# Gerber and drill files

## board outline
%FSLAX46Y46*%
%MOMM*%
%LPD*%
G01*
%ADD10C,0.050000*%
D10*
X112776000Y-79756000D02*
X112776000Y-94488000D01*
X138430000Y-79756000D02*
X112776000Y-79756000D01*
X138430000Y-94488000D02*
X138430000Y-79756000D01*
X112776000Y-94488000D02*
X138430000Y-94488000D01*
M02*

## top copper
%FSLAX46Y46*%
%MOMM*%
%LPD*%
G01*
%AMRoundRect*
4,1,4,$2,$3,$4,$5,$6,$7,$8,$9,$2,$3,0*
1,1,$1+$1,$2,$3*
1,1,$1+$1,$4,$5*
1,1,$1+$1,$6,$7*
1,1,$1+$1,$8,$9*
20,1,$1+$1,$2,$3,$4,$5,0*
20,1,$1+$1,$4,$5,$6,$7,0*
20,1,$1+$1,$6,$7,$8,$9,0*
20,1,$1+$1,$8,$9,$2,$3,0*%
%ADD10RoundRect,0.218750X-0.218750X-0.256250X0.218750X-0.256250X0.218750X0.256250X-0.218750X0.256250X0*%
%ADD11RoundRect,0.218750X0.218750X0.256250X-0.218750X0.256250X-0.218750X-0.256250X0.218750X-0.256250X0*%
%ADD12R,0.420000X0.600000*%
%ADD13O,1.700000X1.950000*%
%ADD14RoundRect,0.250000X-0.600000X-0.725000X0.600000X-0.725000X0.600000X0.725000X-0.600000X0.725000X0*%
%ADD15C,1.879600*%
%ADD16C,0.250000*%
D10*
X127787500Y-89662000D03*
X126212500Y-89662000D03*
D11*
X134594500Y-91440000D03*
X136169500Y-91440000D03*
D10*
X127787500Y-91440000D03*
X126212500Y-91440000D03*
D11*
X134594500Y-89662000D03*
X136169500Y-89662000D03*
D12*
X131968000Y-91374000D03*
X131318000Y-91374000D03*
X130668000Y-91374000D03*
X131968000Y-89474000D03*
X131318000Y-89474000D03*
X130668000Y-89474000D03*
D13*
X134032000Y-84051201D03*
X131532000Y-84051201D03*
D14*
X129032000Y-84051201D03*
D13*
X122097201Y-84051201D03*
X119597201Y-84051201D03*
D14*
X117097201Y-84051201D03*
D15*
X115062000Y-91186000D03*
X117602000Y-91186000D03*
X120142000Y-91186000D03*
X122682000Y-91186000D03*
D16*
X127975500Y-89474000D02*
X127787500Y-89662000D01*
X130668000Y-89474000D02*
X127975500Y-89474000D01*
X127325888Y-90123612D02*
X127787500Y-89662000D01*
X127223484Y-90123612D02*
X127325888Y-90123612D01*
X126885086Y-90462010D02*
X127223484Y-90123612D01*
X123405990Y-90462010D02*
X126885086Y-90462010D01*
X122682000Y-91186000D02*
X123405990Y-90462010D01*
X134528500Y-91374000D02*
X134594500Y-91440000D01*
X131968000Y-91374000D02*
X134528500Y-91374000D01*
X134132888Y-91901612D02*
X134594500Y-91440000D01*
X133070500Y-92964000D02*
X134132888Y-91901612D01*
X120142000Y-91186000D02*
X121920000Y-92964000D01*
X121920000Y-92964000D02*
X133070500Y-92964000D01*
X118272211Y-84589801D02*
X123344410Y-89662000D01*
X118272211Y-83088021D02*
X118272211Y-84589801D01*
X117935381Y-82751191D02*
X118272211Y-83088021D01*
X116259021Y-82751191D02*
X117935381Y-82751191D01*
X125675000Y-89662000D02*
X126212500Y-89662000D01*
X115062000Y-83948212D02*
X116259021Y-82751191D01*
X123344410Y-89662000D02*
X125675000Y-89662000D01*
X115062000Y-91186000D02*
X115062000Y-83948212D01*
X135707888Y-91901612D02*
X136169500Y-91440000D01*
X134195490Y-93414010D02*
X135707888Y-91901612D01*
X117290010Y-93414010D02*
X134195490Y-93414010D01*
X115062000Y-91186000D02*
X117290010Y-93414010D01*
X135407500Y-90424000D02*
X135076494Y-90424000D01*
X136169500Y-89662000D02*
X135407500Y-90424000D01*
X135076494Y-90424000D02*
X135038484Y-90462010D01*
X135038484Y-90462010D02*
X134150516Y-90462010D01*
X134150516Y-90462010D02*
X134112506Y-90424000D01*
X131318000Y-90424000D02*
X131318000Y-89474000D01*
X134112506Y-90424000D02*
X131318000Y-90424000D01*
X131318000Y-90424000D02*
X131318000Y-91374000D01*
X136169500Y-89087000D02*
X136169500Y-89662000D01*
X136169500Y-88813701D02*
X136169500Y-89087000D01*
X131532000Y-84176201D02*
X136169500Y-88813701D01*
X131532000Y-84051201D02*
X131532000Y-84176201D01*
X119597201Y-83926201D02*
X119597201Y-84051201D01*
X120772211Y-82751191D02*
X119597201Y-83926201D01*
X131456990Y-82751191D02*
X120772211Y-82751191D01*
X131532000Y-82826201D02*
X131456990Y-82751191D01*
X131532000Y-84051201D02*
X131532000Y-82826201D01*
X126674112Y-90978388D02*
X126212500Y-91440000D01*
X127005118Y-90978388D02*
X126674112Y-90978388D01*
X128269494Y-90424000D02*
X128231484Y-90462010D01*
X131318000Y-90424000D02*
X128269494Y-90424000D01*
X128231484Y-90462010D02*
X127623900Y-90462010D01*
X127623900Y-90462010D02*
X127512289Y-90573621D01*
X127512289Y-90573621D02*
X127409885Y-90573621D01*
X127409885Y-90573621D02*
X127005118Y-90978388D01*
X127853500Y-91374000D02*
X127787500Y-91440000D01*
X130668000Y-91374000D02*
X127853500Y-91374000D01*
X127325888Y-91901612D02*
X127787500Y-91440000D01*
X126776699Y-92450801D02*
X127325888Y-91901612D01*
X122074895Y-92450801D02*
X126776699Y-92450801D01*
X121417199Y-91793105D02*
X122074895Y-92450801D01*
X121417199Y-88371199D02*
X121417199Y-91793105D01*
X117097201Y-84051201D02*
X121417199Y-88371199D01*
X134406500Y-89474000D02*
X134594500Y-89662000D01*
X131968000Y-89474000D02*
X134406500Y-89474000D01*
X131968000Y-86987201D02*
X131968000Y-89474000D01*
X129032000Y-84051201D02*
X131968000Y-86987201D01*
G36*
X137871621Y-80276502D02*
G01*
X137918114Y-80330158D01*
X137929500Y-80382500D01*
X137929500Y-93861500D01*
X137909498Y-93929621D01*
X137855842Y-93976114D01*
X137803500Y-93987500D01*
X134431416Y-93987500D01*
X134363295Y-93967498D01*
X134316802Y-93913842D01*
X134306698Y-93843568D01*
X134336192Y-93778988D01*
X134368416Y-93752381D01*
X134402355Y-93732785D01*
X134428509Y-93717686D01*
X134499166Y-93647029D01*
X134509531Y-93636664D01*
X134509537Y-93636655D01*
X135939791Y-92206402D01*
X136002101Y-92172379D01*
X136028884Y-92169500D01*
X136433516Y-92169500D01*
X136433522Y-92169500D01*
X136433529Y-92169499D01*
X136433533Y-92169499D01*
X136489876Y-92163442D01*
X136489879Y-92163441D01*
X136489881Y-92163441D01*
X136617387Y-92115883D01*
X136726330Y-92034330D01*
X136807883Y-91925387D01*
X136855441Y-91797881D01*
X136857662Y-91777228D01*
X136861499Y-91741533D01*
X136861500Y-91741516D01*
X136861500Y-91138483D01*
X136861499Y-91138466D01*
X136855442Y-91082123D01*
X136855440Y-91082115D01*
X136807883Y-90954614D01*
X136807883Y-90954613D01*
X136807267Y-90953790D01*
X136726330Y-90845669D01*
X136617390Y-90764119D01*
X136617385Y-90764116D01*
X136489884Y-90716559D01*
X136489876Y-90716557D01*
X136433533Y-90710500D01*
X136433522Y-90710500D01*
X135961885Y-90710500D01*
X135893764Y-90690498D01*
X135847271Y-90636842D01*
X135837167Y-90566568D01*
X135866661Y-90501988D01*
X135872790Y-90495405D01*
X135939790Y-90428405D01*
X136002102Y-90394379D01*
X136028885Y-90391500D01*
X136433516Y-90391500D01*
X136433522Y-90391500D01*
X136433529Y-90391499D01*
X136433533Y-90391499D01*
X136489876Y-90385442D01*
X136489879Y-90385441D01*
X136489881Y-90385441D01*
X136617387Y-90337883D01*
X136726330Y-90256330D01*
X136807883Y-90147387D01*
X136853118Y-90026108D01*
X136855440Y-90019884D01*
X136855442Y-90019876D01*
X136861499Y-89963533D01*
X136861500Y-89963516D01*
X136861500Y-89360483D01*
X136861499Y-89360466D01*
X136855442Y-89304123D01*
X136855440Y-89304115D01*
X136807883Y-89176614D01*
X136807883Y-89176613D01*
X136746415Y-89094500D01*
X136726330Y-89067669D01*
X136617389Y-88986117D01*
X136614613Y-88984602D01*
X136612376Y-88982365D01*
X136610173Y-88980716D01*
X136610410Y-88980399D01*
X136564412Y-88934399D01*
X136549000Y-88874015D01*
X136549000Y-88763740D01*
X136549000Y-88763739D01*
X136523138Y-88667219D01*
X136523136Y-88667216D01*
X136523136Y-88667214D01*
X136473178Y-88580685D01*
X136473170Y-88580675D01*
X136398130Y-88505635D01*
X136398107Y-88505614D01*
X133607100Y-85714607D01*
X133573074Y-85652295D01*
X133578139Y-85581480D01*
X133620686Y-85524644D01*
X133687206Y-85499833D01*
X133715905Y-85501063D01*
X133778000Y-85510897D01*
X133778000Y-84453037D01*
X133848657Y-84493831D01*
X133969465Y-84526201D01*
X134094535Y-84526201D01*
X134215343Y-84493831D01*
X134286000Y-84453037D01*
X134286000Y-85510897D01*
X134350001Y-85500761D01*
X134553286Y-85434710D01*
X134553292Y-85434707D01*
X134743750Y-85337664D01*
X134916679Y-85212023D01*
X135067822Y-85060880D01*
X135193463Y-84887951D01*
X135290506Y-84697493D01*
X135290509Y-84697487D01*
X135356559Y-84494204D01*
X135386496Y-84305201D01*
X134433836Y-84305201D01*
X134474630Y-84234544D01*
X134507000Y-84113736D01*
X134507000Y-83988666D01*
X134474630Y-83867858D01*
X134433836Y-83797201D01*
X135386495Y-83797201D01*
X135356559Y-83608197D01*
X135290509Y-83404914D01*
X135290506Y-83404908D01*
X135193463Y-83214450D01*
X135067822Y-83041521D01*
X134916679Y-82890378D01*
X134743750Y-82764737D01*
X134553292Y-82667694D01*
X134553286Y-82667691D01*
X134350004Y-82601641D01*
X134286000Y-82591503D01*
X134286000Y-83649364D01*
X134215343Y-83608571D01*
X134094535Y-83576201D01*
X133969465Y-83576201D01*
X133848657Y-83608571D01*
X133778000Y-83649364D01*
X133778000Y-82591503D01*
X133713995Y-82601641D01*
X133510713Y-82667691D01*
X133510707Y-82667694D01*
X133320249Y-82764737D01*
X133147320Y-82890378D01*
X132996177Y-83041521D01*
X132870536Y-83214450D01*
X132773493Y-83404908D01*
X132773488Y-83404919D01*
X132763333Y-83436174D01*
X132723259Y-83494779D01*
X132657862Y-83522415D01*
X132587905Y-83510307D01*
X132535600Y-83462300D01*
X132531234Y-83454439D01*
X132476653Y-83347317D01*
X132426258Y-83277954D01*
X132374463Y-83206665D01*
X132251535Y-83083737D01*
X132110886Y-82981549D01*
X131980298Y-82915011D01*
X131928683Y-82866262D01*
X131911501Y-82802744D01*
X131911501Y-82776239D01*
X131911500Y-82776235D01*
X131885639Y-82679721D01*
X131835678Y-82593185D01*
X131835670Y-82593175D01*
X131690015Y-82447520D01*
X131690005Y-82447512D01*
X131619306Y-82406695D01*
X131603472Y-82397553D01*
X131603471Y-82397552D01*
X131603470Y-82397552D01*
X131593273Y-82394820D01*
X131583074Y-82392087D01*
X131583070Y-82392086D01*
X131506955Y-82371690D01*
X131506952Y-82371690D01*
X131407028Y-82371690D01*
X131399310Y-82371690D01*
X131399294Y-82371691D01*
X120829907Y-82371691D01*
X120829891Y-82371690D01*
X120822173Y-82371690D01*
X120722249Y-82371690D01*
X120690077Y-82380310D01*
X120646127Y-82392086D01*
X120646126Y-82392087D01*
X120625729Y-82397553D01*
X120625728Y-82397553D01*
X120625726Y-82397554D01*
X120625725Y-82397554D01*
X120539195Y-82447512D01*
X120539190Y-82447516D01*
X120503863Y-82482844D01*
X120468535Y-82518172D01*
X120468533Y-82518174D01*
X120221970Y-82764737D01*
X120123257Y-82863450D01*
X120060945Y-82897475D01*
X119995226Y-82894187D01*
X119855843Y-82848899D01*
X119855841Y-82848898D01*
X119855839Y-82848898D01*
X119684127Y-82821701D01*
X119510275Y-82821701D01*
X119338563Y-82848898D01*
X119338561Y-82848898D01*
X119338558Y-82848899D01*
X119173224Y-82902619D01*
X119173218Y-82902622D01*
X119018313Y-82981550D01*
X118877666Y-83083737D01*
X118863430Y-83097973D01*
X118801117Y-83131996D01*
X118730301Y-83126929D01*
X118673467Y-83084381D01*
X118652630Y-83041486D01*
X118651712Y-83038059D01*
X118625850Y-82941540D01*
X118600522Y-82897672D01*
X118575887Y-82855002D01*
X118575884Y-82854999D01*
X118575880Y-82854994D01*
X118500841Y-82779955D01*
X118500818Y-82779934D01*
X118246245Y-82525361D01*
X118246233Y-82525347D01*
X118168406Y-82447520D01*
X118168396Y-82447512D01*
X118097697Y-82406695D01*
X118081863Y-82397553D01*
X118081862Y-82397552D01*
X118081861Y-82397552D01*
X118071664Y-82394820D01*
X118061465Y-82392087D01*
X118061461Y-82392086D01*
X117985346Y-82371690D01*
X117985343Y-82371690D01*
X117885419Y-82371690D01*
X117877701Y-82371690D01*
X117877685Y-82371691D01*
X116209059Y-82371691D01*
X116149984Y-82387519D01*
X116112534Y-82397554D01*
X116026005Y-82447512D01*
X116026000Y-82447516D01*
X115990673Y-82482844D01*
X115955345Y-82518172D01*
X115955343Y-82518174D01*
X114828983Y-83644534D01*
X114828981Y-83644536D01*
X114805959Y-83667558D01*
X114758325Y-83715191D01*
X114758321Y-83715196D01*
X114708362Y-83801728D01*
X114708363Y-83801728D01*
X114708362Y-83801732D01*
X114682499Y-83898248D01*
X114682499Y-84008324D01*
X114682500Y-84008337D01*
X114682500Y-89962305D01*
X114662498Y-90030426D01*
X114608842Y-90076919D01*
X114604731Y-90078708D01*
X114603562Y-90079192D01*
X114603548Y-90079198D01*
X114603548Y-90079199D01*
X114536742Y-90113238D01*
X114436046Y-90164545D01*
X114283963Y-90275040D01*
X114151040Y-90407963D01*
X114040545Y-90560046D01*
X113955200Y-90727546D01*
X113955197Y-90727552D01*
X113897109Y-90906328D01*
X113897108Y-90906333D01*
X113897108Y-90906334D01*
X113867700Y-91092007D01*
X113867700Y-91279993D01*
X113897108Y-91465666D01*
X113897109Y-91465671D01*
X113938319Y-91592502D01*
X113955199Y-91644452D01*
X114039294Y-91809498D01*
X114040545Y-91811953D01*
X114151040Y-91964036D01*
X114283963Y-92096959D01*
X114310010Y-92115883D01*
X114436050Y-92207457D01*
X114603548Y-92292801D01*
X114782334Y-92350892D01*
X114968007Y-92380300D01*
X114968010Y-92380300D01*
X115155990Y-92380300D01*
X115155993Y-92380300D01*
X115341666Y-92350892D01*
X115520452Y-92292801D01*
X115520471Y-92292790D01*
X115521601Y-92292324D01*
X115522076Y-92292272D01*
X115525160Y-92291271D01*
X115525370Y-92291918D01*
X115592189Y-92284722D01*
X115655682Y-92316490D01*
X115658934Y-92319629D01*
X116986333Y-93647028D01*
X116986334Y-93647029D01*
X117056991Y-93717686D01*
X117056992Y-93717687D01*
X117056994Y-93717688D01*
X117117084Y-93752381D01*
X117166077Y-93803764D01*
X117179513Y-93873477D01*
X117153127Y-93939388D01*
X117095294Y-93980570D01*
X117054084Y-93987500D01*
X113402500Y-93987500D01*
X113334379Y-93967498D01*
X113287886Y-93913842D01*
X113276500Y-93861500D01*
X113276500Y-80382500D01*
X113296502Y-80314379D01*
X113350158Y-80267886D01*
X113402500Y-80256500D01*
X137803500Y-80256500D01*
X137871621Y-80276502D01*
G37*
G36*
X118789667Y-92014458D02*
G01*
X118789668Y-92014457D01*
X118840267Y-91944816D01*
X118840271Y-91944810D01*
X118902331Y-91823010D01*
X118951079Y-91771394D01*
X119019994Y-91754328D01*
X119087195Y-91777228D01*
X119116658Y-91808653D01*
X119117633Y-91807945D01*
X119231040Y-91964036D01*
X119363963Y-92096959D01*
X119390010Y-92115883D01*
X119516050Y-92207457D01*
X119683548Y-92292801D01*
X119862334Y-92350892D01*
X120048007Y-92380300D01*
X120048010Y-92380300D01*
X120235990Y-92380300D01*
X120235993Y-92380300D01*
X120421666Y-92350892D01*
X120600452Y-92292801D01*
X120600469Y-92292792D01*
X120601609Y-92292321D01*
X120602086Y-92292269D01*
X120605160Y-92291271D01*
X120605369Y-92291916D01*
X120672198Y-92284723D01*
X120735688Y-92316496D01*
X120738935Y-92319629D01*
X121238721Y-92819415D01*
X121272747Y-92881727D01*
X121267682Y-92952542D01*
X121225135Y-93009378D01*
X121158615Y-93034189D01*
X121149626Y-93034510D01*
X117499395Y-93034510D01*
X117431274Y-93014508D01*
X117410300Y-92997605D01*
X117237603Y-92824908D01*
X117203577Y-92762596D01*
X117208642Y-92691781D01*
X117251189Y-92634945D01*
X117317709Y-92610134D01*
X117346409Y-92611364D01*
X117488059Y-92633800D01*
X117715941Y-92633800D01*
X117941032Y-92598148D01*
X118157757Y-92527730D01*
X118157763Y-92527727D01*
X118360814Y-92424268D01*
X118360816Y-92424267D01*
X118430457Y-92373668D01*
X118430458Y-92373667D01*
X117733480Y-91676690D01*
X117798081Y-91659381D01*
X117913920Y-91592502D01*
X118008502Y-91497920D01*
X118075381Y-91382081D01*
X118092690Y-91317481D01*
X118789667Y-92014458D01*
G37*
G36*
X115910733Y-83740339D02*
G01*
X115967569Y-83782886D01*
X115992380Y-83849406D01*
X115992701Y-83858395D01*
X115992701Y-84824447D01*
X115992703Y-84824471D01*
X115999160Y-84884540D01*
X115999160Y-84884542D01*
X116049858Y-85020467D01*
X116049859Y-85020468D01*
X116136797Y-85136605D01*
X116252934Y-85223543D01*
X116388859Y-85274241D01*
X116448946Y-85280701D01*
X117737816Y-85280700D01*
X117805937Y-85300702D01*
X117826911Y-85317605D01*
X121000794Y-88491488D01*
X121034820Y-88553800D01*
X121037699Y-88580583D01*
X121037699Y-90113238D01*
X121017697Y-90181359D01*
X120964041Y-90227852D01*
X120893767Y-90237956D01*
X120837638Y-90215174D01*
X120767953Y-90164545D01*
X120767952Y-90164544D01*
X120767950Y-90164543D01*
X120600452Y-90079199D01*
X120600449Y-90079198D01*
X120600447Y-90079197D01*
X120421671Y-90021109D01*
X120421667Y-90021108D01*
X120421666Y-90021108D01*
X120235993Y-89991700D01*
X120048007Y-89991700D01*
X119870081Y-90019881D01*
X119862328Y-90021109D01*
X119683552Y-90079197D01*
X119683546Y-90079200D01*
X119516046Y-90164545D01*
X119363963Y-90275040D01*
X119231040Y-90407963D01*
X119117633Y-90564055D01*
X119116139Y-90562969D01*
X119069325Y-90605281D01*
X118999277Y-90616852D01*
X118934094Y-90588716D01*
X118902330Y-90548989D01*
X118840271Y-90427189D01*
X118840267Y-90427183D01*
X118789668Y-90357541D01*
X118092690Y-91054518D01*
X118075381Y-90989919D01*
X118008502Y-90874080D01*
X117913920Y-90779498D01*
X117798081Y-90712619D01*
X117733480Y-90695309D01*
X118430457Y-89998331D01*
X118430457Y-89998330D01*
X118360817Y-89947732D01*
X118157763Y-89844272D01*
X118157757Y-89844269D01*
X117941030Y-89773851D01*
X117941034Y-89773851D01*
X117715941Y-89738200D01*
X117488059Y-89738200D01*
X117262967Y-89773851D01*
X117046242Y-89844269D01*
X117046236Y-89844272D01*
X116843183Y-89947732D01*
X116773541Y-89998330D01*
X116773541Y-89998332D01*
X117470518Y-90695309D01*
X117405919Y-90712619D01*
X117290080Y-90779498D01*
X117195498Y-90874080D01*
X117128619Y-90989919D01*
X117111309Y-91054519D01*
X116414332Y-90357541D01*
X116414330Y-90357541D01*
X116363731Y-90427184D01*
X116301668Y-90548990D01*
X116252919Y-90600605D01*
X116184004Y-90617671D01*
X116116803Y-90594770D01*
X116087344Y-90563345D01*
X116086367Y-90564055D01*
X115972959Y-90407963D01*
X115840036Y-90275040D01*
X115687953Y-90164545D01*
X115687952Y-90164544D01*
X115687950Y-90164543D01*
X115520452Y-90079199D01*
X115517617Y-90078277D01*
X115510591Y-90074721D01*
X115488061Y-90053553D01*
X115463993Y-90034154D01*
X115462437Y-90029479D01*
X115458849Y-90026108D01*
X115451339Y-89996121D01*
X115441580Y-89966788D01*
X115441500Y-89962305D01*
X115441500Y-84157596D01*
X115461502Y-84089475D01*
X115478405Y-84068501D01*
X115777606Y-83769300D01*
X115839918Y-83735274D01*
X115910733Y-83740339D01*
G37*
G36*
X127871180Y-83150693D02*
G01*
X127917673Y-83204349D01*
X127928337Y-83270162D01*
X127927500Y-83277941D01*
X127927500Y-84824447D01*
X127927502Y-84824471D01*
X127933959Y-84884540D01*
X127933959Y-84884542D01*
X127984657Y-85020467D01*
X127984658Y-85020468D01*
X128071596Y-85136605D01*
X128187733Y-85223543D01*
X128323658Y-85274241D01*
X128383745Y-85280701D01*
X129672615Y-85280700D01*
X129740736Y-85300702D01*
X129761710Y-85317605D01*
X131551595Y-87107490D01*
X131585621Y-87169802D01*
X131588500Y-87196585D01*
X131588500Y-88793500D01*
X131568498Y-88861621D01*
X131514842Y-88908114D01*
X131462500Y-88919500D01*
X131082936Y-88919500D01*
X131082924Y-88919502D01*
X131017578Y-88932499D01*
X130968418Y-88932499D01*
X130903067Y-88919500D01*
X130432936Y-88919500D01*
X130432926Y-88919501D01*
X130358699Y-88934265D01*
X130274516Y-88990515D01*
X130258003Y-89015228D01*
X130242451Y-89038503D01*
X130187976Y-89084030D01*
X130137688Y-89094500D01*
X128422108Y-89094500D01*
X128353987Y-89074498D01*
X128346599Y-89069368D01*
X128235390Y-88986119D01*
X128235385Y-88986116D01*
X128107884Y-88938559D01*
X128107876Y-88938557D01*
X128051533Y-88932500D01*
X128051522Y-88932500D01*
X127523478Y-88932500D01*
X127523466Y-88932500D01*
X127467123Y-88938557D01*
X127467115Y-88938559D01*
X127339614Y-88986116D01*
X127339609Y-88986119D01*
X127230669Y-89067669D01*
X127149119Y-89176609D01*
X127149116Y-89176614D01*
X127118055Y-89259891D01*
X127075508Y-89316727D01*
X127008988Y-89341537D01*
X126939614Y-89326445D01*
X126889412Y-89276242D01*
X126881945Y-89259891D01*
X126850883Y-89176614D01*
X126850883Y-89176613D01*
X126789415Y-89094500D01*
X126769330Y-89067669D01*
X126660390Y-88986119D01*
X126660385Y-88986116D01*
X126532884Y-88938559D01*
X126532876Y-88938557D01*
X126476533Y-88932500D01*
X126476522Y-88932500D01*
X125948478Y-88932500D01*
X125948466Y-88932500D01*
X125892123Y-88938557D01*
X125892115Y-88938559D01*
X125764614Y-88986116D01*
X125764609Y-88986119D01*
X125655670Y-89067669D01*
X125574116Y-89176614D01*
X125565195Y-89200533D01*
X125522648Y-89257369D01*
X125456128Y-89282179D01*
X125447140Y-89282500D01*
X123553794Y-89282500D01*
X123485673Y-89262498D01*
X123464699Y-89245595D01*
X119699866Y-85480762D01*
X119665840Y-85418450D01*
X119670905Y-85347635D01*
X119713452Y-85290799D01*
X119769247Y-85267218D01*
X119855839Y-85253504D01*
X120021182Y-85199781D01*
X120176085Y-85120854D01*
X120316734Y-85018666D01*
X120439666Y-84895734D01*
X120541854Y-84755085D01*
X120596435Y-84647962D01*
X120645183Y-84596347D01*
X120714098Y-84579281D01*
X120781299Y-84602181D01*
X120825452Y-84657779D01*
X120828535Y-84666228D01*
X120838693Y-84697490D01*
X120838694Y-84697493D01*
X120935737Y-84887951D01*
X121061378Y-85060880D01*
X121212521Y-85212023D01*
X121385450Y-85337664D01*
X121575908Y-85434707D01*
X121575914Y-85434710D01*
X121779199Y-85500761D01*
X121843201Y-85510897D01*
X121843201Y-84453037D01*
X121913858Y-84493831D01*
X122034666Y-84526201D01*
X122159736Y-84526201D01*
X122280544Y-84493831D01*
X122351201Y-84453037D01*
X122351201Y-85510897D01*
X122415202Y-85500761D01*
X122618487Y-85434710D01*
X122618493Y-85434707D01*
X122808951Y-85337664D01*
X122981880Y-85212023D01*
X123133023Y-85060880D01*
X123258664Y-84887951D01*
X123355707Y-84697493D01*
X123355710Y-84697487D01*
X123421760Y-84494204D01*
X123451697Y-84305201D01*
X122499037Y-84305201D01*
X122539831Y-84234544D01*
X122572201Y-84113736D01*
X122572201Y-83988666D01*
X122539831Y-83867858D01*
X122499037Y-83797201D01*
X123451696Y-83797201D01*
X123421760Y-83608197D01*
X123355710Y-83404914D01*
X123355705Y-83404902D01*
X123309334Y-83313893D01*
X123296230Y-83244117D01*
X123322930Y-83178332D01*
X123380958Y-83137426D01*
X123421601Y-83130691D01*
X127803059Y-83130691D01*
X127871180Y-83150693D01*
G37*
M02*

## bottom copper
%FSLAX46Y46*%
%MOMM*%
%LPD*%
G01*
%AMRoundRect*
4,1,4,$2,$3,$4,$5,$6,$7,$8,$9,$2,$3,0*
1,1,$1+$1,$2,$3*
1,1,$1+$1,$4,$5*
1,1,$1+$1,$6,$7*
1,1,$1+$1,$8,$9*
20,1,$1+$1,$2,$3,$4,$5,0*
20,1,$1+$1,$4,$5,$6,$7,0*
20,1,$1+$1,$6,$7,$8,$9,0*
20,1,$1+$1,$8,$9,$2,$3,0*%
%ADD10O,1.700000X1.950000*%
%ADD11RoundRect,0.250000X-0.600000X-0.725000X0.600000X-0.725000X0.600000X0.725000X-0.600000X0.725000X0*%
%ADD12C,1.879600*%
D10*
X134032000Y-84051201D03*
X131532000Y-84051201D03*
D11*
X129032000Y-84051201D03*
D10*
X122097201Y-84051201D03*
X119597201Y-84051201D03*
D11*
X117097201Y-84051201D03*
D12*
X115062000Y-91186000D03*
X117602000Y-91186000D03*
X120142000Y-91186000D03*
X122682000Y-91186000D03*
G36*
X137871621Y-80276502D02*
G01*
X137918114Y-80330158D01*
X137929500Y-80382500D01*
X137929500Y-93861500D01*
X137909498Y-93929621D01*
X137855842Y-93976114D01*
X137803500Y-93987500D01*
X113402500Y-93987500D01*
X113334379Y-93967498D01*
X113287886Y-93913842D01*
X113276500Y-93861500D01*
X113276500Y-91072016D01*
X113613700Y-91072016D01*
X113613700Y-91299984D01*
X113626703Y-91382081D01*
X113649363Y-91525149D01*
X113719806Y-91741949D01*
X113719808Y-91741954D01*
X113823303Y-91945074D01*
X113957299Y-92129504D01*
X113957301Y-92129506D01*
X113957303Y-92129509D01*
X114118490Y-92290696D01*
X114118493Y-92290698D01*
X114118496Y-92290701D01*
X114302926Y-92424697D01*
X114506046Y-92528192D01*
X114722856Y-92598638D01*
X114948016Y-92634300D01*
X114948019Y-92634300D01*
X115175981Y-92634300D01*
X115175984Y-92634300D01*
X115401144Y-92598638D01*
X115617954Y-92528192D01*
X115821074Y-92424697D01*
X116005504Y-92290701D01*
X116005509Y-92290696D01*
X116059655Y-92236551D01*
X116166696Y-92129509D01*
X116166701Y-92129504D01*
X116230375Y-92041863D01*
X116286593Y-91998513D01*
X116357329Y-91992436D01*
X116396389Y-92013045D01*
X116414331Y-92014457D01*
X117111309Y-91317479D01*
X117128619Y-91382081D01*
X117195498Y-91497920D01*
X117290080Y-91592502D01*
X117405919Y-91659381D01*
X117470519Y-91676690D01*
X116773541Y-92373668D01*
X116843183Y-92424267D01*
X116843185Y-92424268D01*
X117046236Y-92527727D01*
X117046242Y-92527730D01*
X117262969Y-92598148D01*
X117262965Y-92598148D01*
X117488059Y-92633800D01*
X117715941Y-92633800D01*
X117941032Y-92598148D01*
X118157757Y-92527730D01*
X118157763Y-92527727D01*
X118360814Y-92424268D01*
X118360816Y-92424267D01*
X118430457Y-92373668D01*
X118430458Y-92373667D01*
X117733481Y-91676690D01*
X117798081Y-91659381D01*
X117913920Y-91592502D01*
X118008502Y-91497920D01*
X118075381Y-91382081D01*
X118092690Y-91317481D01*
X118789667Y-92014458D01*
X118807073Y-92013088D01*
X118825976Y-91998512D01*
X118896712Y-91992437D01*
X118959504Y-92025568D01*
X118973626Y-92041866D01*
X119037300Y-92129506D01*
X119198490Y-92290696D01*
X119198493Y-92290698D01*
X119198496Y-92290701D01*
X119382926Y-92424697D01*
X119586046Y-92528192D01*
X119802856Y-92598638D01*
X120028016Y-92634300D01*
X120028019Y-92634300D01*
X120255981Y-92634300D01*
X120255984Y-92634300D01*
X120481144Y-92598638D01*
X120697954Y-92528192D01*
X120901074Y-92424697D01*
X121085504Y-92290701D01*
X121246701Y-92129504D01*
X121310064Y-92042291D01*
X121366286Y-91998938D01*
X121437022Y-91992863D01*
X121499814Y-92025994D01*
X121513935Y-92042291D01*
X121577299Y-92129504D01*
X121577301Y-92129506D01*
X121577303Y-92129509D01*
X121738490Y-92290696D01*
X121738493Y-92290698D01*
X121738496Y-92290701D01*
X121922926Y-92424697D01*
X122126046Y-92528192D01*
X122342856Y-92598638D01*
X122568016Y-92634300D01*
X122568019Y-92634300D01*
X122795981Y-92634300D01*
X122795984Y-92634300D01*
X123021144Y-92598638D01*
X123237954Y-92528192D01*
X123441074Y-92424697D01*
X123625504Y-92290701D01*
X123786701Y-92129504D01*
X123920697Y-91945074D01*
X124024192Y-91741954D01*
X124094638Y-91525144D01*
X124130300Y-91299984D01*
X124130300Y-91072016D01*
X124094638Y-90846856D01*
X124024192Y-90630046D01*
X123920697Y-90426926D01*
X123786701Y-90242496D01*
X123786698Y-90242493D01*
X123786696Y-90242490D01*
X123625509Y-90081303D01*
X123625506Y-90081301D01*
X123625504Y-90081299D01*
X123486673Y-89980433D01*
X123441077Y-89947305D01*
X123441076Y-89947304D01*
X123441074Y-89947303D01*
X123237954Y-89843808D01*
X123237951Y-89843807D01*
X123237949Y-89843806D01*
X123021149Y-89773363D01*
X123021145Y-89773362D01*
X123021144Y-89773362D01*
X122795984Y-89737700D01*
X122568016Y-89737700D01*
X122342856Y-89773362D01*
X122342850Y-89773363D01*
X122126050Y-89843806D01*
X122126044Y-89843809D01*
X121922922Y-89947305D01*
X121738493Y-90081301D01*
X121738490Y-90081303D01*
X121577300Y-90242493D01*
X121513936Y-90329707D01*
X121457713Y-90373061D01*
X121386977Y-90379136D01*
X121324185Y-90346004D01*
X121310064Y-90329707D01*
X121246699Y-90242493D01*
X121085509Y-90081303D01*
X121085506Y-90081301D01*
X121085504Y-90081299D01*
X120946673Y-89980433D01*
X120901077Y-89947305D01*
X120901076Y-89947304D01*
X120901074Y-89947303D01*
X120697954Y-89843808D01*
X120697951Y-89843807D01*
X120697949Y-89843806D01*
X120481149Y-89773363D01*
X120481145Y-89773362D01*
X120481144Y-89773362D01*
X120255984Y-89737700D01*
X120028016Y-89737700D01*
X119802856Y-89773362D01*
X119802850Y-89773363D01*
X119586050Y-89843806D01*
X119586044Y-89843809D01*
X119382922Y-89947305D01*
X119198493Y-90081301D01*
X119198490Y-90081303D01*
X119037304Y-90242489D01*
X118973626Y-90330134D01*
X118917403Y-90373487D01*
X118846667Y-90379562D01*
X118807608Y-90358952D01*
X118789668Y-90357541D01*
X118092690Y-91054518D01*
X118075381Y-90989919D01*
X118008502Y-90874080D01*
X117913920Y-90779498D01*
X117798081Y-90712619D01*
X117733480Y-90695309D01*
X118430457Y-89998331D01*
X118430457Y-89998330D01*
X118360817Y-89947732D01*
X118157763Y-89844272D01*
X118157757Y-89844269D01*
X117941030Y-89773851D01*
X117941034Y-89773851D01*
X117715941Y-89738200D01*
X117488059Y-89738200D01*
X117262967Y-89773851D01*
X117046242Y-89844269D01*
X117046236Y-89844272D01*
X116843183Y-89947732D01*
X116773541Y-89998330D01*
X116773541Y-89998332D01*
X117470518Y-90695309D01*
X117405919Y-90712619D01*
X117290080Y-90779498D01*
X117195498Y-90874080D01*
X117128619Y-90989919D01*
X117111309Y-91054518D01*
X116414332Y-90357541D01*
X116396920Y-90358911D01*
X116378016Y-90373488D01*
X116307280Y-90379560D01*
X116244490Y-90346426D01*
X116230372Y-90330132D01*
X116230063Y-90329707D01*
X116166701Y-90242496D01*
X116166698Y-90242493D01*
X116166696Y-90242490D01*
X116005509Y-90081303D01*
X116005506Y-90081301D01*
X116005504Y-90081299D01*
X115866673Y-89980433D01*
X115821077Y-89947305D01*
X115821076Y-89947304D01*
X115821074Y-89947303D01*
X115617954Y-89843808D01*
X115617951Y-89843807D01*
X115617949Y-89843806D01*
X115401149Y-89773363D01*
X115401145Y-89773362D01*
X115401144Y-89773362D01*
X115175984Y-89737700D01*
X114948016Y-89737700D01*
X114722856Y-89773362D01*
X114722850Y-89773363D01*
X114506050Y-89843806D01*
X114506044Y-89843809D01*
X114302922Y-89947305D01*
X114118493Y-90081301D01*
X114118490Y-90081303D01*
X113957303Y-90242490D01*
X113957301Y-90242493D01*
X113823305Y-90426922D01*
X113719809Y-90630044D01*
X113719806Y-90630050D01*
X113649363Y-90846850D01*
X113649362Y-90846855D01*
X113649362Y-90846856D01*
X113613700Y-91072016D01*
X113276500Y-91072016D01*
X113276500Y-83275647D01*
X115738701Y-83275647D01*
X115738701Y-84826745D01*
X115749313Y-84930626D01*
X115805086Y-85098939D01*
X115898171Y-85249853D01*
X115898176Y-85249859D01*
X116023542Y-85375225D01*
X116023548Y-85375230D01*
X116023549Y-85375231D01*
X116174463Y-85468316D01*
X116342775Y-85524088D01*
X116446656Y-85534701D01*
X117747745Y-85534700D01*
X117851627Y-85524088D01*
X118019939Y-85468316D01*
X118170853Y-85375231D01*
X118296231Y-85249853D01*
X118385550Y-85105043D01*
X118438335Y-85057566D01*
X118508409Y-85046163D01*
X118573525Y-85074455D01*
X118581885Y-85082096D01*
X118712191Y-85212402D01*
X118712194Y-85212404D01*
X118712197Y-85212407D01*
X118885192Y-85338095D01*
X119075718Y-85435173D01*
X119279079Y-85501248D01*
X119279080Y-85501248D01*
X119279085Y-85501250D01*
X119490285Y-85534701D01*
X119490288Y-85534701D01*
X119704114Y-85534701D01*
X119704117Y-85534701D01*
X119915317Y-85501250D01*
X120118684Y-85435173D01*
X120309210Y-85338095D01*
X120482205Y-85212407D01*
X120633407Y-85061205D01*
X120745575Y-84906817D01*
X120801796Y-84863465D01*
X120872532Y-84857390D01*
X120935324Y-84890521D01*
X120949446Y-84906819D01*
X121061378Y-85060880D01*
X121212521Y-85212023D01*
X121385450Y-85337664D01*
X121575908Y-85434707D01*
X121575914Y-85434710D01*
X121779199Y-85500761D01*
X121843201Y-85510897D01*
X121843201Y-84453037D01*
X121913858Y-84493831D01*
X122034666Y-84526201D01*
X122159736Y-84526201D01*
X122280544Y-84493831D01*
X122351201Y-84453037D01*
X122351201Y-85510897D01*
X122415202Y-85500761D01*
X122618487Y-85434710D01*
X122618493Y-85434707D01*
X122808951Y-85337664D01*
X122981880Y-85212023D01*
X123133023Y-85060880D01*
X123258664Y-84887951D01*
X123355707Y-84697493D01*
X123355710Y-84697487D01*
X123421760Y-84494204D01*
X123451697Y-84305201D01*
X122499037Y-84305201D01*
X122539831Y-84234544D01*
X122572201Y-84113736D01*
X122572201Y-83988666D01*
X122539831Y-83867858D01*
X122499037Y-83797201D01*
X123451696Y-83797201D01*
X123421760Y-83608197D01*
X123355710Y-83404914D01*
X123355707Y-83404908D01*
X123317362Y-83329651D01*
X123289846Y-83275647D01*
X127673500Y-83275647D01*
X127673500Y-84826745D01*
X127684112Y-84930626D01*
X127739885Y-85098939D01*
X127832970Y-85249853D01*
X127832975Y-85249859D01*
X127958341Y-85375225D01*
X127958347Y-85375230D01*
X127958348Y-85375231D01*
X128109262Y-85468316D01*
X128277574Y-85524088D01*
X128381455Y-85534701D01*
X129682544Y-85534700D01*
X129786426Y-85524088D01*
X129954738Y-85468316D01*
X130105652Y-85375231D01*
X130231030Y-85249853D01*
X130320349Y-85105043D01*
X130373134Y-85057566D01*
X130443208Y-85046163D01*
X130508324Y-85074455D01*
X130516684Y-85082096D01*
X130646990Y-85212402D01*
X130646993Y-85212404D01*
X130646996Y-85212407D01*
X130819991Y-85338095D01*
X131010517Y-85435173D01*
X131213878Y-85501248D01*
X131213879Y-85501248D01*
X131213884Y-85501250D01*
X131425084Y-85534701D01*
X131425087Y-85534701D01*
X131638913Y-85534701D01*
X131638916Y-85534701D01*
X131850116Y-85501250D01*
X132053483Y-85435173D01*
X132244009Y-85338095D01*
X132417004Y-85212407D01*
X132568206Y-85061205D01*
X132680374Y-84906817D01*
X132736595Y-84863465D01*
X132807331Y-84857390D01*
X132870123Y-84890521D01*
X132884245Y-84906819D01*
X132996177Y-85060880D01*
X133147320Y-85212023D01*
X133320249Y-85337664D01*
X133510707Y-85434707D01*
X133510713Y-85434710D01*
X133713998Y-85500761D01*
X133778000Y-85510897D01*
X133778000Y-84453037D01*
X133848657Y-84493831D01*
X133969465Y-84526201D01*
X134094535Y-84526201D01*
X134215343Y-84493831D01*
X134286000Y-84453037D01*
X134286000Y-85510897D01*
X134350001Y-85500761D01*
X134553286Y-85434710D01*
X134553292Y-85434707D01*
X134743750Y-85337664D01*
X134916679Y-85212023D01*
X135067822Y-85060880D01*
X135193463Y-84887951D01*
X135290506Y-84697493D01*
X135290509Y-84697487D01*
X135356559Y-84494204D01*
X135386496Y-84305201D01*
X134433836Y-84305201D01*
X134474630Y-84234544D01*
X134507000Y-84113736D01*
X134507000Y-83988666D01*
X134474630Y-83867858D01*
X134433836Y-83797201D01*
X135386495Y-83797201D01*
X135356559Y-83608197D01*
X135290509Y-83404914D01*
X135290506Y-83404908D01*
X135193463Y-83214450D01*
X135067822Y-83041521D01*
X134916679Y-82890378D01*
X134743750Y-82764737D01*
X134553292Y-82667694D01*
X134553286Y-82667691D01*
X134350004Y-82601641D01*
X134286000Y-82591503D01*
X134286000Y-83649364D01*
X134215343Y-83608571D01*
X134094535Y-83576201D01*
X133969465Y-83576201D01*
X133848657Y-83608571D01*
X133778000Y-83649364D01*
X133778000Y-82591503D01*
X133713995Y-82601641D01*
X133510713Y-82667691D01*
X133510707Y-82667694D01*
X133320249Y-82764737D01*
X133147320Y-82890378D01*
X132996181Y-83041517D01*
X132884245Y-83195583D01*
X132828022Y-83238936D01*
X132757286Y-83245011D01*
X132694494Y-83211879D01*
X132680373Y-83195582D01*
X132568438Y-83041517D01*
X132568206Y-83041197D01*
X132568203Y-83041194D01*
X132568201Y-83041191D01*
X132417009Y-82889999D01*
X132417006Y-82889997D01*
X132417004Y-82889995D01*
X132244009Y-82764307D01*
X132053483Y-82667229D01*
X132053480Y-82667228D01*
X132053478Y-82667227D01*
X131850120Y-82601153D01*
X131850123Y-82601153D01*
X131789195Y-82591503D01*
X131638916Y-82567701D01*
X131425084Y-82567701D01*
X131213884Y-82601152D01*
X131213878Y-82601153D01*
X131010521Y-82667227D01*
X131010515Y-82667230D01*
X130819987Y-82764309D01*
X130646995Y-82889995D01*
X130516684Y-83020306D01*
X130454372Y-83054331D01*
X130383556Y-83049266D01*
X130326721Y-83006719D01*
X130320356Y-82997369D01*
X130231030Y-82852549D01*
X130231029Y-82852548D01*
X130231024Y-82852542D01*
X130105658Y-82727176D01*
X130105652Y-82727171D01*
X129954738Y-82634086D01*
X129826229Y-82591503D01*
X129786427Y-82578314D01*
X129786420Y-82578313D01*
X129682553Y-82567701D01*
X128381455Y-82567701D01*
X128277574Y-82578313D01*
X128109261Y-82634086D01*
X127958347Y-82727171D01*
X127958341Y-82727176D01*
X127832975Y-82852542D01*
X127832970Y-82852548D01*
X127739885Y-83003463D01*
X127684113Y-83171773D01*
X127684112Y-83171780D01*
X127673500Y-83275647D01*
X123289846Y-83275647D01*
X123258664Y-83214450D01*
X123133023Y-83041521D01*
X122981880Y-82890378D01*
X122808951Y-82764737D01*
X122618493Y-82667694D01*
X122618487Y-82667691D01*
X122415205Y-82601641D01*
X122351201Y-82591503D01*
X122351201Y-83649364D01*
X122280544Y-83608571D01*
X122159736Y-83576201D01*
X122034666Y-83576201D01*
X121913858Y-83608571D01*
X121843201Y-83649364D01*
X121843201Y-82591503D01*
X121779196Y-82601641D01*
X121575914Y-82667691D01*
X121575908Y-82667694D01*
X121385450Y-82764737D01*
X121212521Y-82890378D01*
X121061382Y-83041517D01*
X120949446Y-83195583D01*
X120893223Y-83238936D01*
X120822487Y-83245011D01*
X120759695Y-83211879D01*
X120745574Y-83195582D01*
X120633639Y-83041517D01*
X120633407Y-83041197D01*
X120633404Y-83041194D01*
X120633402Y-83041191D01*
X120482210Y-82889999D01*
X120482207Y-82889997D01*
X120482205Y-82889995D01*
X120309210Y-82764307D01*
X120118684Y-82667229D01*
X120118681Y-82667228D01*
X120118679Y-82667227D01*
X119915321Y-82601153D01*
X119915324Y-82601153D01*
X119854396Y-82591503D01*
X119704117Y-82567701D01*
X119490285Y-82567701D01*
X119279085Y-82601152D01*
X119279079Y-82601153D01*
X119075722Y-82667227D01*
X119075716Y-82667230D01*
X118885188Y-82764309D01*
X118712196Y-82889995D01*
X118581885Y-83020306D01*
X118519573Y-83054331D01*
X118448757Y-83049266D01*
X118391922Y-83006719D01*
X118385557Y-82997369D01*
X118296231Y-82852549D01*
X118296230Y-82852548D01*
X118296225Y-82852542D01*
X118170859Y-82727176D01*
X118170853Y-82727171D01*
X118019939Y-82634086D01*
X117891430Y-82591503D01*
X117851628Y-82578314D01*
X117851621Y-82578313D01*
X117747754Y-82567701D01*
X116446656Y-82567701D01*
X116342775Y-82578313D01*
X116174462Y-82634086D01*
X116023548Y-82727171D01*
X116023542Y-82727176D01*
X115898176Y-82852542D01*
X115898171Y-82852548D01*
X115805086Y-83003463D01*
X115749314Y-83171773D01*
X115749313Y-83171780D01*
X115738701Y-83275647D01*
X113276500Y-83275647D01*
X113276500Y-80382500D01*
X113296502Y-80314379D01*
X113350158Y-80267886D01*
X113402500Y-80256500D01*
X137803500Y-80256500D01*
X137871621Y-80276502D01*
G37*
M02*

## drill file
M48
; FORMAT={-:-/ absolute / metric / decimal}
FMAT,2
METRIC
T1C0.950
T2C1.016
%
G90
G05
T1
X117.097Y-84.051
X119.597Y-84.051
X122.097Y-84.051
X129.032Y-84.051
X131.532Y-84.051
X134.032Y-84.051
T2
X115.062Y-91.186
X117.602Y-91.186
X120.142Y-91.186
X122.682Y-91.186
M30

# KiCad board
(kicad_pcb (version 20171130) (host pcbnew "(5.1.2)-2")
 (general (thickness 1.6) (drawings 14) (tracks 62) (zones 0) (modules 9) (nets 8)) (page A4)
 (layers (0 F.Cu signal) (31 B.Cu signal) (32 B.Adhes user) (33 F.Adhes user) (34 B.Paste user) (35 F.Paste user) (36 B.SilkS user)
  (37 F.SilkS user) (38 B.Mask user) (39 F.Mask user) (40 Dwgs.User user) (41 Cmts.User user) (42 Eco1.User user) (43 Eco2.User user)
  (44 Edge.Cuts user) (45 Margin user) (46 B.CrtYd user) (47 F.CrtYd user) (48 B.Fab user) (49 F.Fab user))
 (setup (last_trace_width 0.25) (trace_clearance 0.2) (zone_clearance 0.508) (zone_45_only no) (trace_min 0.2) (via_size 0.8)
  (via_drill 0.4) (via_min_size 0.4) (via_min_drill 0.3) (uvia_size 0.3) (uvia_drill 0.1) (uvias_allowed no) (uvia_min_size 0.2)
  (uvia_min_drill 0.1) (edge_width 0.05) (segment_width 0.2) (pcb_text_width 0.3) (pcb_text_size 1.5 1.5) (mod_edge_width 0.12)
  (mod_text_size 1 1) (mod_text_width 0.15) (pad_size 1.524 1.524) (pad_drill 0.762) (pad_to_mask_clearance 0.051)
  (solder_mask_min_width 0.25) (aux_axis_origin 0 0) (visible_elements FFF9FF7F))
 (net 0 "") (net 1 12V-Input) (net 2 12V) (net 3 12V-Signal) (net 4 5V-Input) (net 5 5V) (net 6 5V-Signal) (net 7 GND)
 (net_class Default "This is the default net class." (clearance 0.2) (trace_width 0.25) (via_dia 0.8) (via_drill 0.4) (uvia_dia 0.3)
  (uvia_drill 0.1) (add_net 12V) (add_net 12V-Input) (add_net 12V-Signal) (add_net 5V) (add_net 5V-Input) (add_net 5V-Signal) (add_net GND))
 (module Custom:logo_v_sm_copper (layer B.Cu) (at 131.318 89.408 180)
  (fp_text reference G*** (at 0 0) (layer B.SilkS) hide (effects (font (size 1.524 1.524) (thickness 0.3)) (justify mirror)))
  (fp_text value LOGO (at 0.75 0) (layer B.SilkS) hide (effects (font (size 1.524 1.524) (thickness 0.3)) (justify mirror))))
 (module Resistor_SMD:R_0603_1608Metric (layer F.Cu) (at 127 89.662)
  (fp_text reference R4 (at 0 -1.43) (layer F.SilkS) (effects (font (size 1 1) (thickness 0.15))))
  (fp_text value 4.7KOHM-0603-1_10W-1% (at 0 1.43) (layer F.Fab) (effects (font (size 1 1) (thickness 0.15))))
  (pad 2 smd roundrect (at 0.7875 0) (size 0.875 0.95) (layers F.Cu F.Paste F.Mask) (roundrect_rratio 0.25) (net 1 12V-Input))
  (pad 1 smd roundrect (at -0.7875 0) (size 0.875 0.95) (layers F.Cu F.Paste F.Mask) (roundrect_rratio 0.25) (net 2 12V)))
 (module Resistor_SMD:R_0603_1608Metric (layer F.Cu) (at 135.382 91.44 180)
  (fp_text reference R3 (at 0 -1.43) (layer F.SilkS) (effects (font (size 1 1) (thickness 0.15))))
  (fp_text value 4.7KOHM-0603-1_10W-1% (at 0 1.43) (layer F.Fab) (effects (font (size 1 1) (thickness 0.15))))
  (pad 2 smd roundrect (at 0.7875 0 180) (size 0.875 0.95) (layers F.Cu F.Paste F.Mask) (roundrect_rratio 0.25) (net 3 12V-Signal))
  (pad 1 smd roundrect (at -0.7875 0 180) (size 0.875 0.95) (layers F.Cu F.Paste F.Mask) (roundrect_rratio 0.25) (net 2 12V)))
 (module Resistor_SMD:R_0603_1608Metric (layer F.Cu) (at 127 91.44)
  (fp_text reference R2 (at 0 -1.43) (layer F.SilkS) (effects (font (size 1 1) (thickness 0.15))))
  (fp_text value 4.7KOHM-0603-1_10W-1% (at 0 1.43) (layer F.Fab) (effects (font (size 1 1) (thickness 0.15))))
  (pad 2 smd roundrect (at 0.7875 0) (size 0.875 0.95) (layers F.Cu F.Paste F.Mask) (roundrect_rratio 0.25) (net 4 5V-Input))
  (pad 1 smd roundrect (at -0.7875 0) (size 0.875 0.95) (layers F.Cu F.Paste F.Mask) (roundrect_rratio 0.25) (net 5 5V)))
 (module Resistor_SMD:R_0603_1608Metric (layer F.Cu) (at 135.382 89.662 180)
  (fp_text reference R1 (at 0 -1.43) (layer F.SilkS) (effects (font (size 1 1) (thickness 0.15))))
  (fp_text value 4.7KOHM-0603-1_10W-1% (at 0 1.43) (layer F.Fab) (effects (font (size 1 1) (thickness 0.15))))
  (pad 2 smd roundrect (at 0.7875 0 180) (size 0.875 0.95) (layers F.Cu F.Paste F.Mask) (roundrect_rratio 0.25) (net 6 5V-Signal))
  (pad 1 smd roundrect (at -0.7875 0 180) (size 0.875 0.95) (layers F.Cu F.Paste F.Mask) (roundrect_rratio 0.25) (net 5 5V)))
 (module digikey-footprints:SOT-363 (layer F.Cu) (at 131.318 90.424)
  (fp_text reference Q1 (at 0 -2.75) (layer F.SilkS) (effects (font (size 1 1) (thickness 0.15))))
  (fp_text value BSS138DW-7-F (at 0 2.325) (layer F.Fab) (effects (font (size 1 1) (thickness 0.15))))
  (pad 3 smd rect (at 0.65 0.95) (size 0.42 0.6) (layers F.Cu F.Paste F.Mask) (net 3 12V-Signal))
  (pad 2 smd rect (at 0 0.95) (size 0.42 0.6) (layers F.Cu F.Paste F.Mask) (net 5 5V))
  (pad 1 smd rect (at -0.65 0.95) (size 0.42 0.6) (layers F.Cu F.Paste F.Mask) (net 4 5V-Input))
  (pad 4 smd rect (at 0.65 -0.95) (size 0.42 0.6) (layers F.Cu F.Paste F.Mask) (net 6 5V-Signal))
  (pad 5 smd rect (at 0 -0.95) (size 0.42 0.6) (layers F.Cu F.Paste F.Mask) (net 5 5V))
  (pad 6 smd rect (at -0.65 -0.95) (size 0.42 0.6) (layers F.Cu F.Paste F.Mask) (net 1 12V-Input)))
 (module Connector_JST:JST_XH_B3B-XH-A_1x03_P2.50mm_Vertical (layer F.Cu) (at 129.032 84.051201)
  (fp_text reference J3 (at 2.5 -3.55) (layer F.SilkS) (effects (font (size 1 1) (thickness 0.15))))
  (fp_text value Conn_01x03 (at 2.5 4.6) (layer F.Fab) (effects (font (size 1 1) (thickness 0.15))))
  (pad 3 thru_hole oval (at 5 0) (size 1.7 1.95) (drill 0.95) (layers *.Cu *.Mask) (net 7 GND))
  (pad 2 thru_hole oval (at 2.5 0) (size 1.7 1.95) (drill 0.95) (layers *.Cu *.Mask) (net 5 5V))
  (pad 1 thru_hole roundrect (at 0 0) (size 1.7 1.95) (drill 0.95) (layers *.Cu *.Mask) (roundrect_rratio 0.147059) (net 6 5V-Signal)))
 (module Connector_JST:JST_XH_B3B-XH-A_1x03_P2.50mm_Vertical (layer F.Cu) (at 117.097201 84.051201)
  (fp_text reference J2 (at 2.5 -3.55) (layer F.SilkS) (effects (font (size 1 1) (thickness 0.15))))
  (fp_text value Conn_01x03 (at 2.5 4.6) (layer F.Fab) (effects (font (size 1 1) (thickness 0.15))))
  (pad 3 thru_hole oval (at 5 0) (size 1.7 1.95) (drill 0.95) (layers *.Cu *.Mask) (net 7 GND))
  (pad 2 thru_hole oval (at 2.5 0) (size 1.7 1.95) (drill 0.95) (layers *.Cu *.Mask) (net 5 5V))
  (pad 1 thru_hole roundrect (at 0 0) (size 1.7 1.95) (drill 0.95) (layers *.Cu *.Mask) (roundrect_rratio 0.147059) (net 4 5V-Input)))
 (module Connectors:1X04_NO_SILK (layer F.Cu) (at 115.062 91.186)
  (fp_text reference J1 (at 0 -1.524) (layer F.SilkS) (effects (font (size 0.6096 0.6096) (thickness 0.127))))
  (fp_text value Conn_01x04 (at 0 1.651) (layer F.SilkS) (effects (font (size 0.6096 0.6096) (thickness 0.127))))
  (pad 1 thru_hole circle (at 0 0) (size 1.8796 1.8796) (drill 1.016) (layers *.Cu *.Mask) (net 2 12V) (solder_mask_margin 0.1016))
  (pad 2 thru_hole circle (at 2.54 0) (size 1.8796 1.8796) (drill 1.016) (layers *.Cu *.Mask) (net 7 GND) (solder_mask_margin 0.1016))
  (pad 3 thru_hole circle (at 5.08 0) (size 1.8796 1.8796) (drill 1.016) (layers *.Cu *.Mask) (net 3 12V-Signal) (solder_mask_margin 0.1016))
  (pad 4 thru_hole circle (at 7.62 0) (size 1.8796 1.8796) (drill 1.016) (layers *.Cu *.Mask) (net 1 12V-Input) (solder_mask_margin 0.1016)))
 (gr_line (start 112.776 79.756) (end 112.776 94.488) (layer Edge.Cuts) (width 0.05))
 (gr_line (start 138.43 79.756) (end 112.776 79.756) (layer Edge.Cuts) (width 0.05))
 (gr_line (start 138.43 94.488) (end 138.43 79.756) (layer Edge.Cuts) (width 0.05))
 (gr_line (start 112.776 94.488) (end 138.43 94.488) (layer Edge.Cuts) (width 0.05))
 (segment (start 127.9755 89.474) (end 127.7875 89.662) (width 0.25) (layer F.Cu) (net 1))
 (segment (start 130.668 89.474) (end 127.9755 89.474) (width 0.25) (layer F.Cu) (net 1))
 (segment (start 127.325888 90.123612) (end 127.7875 89.662) (width 0.25) (layer F.Cu) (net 1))
 (segment (start 127.223484 90.123612) (end 127.325888 90.123612) (width 0.25) (layer F.Cu) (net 1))
 (segment (start 126.885086 90.46201) (end 127.223484 90.123612) (width 0.25) (layer F.Cu) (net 1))
 (segment (start 123.40599 90.46201) (end 126.885086 90.46201) (width 0.25) (layer F.Cu) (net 1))
 (segment (start 122.682 91.186) (end 123.40599 90.46201) (width 0.25) (layer F.Cu) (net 1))
 (segment (start 134.5285 91.374) (end 134.5945 91.44) (width 0.25) (layer F.Cu) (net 3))
 (segment (start 131.968 91.374) (end 134.5285 91.374) (width 0.25) (layer F.Cu) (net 3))
 (segment (start 134.132888 91.901612) (end 134.5945 91.44) (width 0.25) (layer F.Cu) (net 3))
 (segment (start 133.0705 92.964) (end 134.132888 91.901612) (width 0.25) (layer F.Cu) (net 3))
 (segment (start 120.142 91.186) (end 121.92 92.964) (width 0.25) (layer F.Cu) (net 3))
 (segment (start 121.92 92.964) (end 133.0705 92.964) (width 0.25) (layer F.Cu) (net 3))
 (segment (start 118.272211 84.589801) (end 123.34441 89.662) (width 0.25) (layer F.Cu) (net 2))
 (segment (start 118.272211 83.088021) (end 118.272211 84.589801) (width 0.25) (layer F.Cu) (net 2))
 (segment (start 117.935381 82.751191) (end 118.272211 83.088021) (width 0.25) (layer F.Cu) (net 2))
 (segment (start 116.259021 82.751191) (end 117.935381 82.751191) (width 0.25) (layer F.Cu) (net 2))
 (segment (start 125.675 89.662) (end 126.2125 89.662) (width 0.25) (layer F.Cu) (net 2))
 (segment (start 115.062 83.948212) (end 116.259021 82.751191) (width 0.25) (layer F.Cu) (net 2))
 (segment (start 123.34441 89.662) (end 125.675 89.662) (width 0.25) (layer F.Cu) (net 2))
 (segment (start 115.062 91.186) (end 115.062 83.948212) (width 0.25) (layer F.Cu) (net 2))
 (segment (start 135.707888 91.901612) (end 136.1695 91.44) (width 0.25) (layer F.Cu) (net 2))
 (segment (start 134.19549 93.41401) (end 135.707888 91.901612) (width 0.25) (layer F.Cu) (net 2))
 (segment (start 117.29001 93.41401) (end 134.19549 93.41401) (width 0.25) (layer F.Cu) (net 2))
 (segment (start 115.062 91.186) (end 117.29001 93.41401) (width 0.25) (layer F.Cu) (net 2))
 (segment (start 135.4075 90.424) (end 135.076494 90.424) (width 0.25) (layer F.Cu) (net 5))
 (segment (start 136.1695 89.662) (end 135.4075 90.424) (width 0.25) (layer F.Cu) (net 5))
 (segment (start 135.076494 90.424) (end 135.038484 90.46201) (width 0.25) (layer F.Cu) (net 5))
 (segment (start 135.038484 90.46201) (end 134.150516 90.46201) (width 0.25) (layer F.Cu) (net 5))
 (segment (start 134.150516 90.46201) (end 134.112506 90.424) (width 0.25) (layer F.Cu) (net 5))
 (segment (start 131.318 90.424) (end 131.318 89.474) (width 0.25) (layer F.Cu) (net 5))
 (segment (start 134.112506 90.424) (end 131.318 90.424) (width 0.25) (layer F.Cu) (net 5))
 (segment (start 131.318 90.424) (end 131.318 91.374) (width 0.25) (layer F.Cu) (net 5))
 (segment (start 136.1695 89.087) (end 136.1695 89.662) (width 0.25) (layer F.Cu) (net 5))
 (segment (start 136.1695 88.813701) (end 136.1695 89.087) (width 0.25) (layer F.Cu) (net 5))
 (segment (start 131.532 84.176201) (end 136.1695 88.813701) (width 0.25) (layer F.Cu) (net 5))
 (segment (start 131.532 84.051201) (end 131.532 84.176201) (width 0.25) (layer F.Cu) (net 5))
 (segment (start 119.597201 83.926201) (end 119.597201 84.051201) (width 0.25) (layer F.Cu) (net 5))
 (segment (start 120.772211 82.751191) (end 119.597201 83.926201) (width 0.25) (layer F.Cu) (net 5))
 (segment (start 131.45699 82.751191) (end 120.772211 82.751191) (width 0.25) (layer F.Cu) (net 5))
 (segment (start 131.532 82.826201) (end 131.45699 82.751191) (width 0.25) (layer F.Cu) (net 5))
 (segment (start 131.532 84.051201) (end 131.532 82.826201) (width 0.25) (layer F.Cu) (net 5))
 (segment (start 126.674112 90.978388) (end 126.2125 91.44) (width 0.25) (layer F.Cu) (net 5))
 (segment (start 127.005118 90.978388) (end 126.674112 90.978388) (width 0.25) (layer F.Cu) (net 5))
 (segment (start 128.269494 90.424) (end 128.231484 90.46201) (width 0.25) (layer F.Cu) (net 5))
 (segment (start 131.318 90.424) (end 128.269494 90.424) (width 0.25) (layer F.Cu) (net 5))
 (segment (start 128.231484 90.46201) (end 127.6239 90.46201) (width 0.25) (layer F.Cu) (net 5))
 (segment (start 127.6239 90.46201) (end 127.512289 90.573621) (width 0.25) (layer F.Cu) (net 5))
 (segment (start 127.512289 90.573621) (end 127.409885 90.573621) (width 0.25) (layer F.Cu) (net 5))
 (segment (start 127.409885 90.573621) (end 127.005118 90.978388) (width 0.25) (layer F.Cu) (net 5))
 (segment (start 127.8535 91.374) (end 127.7875 91.44) (width 0.25) (layer F.Cu) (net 4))
 (segment (start 130.668 91.374) (end 127.8535 91.374) (width 0.25) (layer F.Cu) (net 4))
 (segment (start 127.325888 91.901612) (end 127.7875 91.44) (width 0.25) (layer F.Cu) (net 4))
 (segment (start 126.776699 92.450801) (end 127.325888 91.901612) (width 0.25) (layer F.Cu) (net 4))
 (segment (start 122.074895 92.450801) (end 126.776699 92.450801) (width 0.25) (layer F.Cu) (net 4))
 (segment (start 121.417199 91.793105) (end 122.074895 92.450801) (width 0.25) (layer F.Cu) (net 4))
 (segment (start 121.417199 88.371199) (end 121.417199 91.793105) (width 0.25) (layer F.Cu) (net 4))
 (segment (start 117.097201 84.051201) (end 121.417199 88.371199) (width 0.25) (layer F.Cu) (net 4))
 (segment (start 134.4065 89.474) (end 134.5945 89.662) (width 0.25) (layer F.Cu) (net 6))
 (segment (start 131.968 89.474) (end 134.4065 89.474) (width 0.25) (layer F.Cu) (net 6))
 (segment (start 131.968 86.987201) (end 131.968 89.474) (width 0.25) (layer F.Cu) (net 6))
 (segment (start 129.032 84.051201) (end 131.968 86.987201) (width 0.25) (layer F.Cu) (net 6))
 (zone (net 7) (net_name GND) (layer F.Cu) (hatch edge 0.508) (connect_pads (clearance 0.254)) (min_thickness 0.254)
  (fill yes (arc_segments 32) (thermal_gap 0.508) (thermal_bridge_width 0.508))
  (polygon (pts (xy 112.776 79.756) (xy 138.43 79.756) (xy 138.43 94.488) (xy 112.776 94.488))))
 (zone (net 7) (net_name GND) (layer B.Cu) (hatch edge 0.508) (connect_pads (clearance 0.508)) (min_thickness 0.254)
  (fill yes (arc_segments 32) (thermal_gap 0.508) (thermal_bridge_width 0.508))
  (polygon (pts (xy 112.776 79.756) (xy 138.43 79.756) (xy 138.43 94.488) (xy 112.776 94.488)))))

